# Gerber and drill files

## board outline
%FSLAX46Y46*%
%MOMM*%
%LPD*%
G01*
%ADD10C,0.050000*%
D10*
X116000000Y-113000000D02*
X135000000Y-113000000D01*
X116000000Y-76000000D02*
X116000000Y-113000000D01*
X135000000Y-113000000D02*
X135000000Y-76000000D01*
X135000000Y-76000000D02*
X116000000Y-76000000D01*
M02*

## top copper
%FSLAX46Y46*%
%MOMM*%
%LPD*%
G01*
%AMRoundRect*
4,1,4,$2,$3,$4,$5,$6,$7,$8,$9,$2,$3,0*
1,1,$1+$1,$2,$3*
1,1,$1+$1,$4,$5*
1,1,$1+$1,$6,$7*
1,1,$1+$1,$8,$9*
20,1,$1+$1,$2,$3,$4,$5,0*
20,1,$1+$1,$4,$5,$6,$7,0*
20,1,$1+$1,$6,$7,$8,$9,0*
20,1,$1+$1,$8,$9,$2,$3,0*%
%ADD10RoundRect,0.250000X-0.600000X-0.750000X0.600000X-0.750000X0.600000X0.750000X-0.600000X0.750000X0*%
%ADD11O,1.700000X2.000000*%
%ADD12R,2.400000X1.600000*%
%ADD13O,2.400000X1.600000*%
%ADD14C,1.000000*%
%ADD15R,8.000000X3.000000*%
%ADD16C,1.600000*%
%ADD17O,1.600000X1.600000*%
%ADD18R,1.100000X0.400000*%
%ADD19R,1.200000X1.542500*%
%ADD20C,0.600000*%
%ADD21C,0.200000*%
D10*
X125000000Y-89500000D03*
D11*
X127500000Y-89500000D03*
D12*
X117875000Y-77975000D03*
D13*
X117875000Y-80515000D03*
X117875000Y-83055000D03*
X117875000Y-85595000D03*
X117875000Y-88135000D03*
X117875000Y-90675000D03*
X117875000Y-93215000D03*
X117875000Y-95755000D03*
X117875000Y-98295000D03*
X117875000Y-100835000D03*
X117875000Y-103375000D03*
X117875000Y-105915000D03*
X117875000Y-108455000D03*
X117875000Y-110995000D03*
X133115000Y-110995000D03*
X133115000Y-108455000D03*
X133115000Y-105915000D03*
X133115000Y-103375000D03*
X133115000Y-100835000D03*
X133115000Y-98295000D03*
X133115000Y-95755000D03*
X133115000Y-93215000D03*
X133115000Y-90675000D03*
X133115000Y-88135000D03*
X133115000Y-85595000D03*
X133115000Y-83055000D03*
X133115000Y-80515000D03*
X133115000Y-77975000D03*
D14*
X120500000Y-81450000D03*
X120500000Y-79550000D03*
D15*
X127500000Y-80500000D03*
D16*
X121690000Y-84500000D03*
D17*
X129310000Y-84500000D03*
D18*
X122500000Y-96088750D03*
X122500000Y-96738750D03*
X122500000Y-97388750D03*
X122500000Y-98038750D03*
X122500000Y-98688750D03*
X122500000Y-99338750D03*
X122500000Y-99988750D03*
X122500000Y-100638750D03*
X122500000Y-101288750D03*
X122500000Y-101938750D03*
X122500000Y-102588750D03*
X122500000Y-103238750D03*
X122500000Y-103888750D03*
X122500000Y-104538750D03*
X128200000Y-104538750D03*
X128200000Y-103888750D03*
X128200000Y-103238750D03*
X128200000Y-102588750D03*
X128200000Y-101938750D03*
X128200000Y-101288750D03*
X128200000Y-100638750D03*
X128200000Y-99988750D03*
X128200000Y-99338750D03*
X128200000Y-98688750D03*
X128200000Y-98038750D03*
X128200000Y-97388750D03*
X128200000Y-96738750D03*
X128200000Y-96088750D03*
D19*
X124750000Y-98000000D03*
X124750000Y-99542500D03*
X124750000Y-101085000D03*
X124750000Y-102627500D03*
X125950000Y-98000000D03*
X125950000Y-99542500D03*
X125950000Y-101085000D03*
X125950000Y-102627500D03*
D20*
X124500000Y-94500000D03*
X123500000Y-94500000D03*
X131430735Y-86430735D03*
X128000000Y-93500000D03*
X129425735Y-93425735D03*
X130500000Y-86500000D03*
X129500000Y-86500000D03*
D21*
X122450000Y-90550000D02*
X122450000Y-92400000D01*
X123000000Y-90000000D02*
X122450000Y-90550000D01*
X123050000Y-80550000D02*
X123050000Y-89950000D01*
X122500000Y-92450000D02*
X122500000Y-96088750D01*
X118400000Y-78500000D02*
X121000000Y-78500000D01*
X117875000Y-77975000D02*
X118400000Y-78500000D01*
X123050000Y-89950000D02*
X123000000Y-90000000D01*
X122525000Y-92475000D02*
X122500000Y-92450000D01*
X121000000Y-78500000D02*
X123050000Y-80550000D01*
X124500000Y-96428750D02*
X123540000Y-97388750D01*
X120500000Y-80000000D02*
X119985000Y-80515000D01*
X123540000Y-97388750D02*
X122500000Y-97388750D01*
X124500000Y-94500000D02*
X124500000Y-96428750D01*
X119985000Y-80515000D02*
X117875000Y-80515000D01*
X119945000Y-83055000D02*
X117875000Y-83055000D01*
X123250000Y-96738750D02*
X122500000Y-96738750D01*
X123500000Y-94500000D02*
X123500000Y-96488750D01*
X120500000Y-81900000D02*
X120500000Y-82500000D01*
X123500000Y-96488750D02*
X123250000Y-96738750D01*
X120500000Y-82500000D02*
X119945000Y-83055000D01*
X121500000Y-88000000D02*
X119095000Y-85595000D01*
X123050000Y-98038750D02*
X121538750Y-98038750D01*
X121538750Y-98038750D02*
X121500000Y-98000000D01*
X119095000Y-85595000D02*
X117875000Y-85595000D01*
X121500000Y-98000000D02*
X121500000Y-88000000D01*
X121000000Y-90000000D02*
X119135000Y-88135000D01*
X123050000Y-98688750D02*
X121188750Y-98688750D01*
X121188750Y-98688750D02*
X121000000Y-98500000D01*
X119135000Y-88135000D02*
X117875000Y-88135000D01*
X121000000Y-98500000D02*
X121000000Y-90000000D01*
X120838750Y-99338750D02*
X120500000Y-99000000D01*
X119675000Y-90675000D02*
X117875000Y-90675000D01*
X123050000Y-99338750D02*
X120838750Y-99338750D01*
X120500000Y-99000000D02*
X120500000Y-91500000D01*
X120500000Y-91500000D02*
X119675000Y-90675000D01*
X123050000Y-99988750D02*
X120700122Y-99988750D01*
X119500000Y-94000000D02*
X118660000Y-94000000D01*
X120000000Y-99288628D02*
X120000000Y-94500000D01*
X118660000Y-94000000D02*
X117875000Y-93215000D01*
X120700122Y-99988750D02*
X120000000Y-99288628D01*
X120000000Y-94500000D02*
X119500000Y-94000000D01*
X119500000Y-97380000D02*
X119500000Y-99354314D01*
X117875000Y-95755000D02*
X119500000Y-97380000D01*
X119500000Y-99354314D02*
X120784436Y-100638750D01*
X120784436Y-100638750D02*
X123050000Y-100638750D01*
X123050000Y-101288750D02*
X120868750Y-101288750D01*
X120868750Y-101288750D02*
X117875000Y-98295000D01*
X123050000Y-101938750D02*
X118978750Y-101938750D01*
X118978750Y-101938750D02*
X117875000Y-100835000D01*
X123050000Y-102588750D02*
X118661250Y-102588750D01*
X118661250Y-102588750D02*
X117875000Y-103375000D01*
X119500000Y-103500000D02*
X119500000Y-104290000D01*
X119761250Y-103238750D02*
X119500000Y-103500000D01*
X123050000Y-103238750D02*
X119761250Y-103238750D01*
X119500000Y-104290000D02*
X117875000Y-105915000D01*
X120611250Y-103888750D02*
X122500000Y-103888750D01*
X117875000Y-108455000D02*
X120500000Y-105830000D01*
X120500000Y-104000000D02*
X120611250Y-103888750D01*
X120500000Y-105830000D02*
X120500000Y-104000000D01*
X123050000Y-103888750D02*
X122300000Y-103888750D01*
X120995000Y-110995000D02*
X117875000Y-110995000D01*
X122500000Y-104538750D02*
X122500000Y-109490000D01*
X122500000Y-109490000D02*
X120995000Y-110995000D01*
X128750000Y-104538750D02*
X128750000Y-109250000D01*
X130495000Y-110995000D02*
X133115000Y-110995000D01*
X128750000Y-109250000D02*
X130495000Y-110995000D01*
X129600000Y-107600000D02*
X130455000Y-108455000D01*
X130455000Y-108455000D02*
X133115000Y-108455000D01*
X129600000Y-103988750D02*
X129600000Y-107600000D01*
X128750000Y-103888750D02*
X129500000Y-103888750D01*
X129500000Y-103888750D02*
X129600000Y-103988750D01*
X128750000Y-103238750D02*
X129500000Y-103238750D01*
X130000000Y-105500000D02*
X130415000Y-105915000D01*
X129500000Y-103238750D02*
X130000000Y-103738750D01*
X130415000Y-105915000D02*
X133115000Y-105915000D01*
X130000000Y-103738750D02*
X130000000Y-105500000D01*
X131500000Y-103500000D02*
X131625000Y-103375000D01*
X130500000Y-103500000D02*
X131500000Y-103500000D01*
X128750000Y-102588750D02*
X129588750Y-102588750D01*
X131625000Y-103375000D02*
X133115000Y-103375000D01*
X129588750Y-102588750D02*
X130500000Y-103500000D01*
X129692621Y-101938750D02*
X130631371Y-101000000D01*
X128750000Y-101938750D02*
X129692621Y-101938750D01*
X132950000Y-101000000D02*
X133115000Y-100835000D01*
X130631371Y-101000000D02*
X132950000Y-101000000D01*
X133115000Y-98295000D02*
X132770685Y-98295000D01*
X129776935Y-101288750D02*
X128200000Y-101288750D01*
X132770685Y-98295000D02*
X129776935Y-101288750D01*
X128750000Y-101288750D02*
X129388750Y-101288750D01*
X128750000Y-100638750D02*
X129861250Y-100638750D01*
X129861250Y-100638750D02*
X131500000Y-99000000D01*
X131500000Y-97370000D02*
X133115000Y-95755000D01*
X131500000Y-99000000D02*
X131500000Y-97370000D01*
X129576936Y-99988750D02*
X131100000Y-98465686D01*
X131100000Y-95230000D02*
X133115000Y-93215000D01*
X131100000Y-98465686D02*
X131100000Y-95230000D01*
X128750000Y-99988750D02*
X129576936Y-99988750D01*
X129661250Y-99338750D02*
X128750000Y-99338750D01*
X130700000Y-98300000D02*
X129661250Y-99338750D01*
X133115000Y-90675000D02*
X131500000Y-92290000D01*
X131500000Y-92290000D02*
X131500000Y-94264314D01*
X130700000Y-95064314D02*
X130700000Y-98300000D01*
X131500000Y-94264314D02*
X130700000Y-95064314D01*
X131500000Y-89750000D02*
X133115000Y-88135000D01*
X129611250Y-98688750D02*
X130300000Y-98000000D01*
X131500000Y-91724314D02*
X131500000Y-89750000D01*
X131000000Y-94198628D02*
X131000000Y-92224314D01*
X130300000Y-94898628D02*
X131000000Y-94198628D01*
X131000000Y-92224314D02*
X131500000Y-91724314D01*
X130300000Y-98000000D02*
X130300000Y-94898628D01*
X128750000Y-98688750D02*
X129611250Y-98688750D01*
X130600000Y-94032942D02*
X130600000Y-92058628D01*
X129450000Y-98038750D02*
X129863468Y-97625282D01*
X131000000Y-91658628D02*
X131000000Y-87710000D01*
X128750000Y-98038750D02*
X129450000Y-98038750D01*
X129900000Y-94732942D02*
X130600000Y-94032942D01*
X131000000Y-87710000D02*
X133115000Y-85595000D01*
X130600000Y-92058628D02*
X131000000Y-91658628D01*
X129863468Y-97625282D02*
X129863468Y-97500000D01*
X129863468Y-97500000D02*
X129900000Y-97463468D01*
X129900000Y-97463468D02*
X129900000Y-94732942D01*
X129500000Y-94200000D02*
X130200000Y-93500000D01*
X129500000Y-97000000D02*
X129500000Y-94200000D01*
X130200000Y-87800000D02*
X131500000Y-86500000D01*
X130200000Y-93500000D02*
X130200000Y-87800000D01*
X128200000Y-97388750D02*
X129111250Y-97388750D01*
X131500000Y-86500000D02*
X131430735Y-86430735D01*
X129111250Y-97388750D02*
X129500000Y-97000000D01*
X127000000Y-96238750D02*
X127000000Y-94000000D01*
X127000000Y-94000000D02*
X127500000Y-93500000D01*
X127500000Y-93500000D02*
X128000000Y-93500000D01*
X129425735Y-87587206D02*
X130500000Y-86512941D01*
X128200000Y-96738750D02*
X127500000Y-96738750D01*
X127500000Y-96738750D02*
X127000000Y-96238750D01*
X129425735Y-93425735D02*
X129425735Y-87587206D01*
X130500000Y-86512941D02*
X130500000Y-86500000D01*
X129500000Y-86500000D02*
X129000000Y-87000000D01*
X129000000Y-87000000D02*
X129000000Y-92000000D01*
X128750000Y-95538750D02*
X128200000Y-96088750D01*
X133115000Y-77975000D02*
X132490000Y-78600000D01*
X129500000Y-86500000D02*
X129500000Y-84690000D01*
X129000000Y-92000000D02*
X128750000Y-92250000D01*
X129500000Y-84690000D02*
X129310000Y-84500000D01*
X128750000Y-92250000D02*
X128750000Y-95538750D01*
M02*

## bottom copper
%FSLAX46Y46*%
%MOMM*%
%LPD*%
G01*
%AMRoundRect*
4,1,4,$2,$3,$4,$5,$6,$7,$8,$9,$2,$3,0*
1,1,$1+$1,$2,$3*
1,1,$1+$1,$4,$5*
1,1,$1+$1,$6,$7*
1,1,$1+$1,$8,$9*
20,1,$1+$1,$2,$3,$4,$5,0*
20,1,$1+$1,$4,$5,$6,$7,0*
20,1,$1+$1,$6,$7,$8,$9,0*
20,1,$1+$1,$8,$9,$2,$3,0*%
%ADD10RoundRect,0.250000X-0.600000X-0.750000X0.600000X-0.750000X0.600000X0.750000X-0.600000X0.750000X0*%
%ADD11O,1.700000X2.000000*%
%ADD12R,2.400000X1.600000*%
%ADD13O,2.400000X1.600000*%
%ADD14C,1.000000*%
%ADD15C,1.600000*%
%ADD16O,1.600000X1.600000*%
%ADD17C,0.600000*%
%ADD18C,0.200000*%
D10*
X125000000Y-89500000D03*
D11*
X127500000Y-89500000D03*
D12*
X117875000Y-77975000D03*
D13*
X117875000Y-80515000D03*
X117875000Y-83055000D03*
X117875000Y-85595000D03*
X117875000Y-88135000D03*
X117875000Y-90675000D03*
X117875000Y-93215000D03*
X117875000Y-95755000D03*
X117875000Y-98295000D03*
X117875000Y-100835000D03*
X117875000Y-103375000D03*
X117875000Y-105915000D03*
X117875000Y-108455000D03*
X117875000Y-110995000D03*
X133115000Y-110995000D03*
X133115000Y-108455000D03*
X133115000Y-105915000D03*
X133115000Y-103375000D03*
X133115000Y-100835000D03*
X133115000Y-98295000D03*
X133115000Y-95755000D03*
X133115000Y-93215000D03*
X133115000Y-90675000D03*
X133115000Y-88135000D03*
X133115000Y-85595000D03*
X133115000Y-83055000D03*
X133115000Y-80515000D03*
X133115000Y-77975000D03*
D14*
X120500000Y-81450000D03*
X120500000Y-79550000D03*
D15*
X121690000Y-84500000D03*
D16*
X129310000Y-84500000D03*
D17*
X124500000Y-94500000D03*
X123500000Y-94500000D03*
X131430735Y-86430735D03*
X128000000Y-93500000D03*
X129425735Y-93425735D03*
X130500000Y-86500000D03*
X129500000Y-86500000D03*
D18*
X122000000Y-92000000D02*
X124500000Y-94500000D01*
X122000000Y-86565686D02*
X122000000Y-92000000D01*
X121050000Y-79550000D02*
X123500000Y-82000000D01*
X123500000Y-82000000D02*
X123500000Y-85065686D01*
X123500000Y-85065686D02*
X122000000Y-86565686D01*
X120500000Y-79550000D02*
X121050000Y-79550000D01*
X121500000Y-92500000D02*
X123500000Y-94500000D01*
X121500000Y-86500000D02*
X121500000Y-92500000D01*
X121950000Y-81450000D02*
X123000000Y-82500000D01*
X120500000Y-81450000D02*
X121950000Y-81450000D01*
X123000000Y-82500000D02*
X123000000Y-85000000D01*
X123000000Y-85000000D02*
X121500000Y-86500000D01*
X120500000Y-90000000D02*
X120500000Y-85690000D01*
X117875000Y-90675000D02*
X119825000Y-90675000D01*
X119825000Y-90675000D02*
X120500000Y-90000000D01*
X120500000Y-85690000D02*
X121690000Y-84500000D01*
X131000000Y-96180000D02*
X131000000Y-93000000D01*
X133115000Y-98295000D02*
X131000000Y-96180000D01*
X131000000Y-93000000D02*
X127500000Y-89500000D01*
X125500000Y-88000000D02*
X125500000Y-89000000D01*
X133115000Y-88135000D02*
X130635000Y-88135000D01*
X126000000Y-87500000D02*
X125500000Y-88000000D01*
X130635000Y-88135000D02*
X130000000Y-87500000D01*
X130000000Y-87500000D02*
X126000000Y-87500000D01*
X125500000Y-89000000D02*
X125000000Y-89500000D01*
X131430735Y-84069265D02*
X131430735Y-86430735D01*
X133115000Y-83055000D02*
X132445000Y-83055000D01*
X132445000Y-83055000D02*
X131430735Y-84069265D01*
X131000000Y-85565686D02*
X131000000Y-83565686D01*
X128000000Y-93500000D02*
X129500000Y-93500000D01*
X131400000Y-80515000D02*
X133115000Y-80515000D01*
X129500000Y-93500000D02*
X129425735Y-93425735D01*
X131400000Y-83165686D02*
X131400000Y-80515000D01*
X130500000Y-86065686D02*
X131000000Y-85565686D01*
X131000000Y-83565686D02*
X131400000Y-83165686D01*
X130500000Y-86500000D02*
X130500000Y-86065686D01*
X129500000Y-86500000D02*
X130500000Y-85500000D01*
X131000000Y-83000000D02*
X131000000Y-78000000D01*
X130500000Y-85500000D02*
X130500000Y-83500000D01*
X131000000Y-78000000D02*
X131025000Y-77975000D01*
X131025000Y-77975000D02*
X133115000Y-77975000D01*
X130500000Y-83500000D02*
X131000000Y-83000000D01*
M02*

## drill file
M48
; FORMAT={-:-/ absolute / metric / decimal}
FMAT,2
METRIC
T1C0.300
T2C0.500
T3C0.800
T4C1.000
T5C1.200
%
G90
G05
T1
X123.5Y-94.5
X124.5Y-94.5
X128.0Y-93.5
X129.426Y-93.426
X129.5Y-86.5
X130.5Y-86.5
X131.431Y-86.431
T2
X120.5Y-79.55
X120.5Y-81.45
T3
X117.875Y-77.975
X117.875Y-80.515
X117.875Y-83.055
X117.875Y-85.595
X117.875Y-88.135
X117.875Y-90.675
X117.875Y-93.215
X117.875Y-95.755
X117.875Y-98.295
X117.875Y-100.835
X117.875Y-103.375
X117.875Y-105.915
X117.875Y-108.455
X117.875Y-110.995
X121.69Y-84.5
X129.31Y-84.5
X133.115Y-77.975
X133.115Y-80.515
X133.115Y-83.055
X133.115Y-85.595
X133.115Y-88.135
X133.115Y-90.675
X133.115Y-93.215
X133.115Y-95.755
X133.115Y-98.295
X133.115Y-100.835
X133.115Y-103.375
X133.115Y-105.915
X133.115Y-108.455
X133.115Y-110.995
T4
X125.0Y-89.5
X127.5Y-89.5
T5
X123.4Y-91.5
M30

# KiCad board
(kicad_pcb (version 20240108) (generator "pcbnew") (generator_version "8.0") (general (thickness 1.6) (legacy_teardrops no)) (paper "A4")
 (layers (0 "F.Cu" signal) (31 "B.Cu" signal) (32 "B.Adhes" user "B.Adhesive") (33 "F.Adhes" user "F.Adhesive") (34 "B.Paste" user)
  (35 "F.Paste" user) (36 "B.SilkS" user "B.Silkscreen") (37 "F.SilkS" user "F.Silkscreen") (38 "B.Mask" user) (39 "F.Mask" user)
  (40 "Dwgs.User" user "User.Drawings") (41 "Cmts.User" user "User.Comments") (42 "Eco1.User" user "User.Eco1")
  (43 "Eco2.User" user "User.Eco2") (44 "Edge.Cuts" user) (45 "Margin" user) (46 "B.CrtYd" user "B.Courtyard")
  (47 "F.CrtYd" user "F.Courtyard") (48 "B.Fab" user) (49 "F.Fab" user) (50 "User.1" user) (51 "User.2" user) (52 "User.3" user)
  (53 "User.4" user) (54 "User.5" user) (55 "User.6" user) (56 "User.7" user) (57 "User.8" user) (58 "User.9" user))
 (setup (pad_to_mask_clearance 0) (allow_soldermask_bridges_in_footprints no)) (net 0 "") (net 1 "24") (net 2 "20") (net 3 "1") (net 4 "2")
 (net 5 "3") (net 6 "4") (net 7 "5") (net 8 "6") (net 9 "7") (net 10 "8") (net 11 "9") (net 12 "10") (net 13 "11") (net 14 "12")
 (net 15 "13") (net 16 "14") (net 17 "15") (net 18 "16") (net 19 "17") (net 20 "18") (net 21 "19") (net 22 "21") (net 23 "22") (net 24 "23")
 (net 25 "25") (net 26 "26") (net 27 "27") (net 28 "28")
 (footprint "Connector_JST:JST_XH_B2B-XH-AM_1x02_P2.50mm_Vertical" (layer "F.Cu") (at 125 89.5)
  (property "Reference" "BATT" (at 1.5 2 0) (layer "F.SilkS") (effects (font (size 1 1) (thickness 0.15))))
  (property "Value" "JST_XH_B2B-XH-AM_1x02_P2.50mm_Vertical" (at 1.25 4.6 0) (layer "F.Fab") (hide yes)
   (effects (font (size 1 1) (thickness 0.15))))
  (pad "" np_thru_hole circle (at -1.6 2) (size 1.2 1.2) (drill 1.2) (layers "*.Cu" "*.Mask"))
  (pad "1" thru_hole roundrect (at 0 0) (size 1.7 2) (drill 1) (layers "*.Cu" "*.Mask") (remove_unused_layers no)
   (roundrect_rratio 0.147059) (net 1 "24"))
  (pad "2" thru_hole oval (at 2.5 0) (size 1.7 2) (drill 1) (layers "*.Cu" "*.Mask") (remove_unused_layers no) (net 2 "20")))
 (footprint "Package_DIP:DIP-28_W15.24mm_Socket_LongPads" (layer "F.Cu") (at 117.875 77.975)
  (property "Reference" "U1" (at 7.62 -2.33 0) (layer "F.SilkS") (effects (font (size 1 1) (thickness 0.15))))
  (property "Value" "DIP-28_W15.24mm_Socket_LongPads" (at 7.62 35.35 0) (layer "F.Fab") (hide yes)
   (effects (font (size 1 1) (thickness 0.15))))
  (pad "1" thru_hole rect (at 0 0) (size 2.4 1.6) (drill 0.8) (layers "*.Cu" "*.Mask") (remove_unused_layers no) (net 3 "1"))
  (pad "2" thru_hole oval (at 0 2.54) (size 2.4 1.6) (drill 0.8) (layers "*.Cu" "*.Mask") (remove_unused_layers no) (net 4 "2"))
  (pad "3" thru_hole oval (at 0 5.08) (size 2.4 1.6) (drill 0.8) (layers "*.Cu" "*.Mask") (remove_unused_layers no) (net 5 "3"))
  (pad "4" thru_hole oval (at 0 7.62) (size 2.4 1.6) (drill 0.8) (layers "*.Cu" "*.Mask") (remove_unused_layers no) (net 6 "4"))
  (pad "5" thru_hole oval (at 0 10.16) (size 2.4 1.6) (drill 0.8) (layers "*.Cu" "*.Mask") (remove_unused_layers no) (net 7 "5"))
  (pad "6" thru_hole oval (at 0 12.7) (size 2.4 1.6) (drill 0.8) (layers "*.Cu" "*.Mask") (remove_unused_layers no) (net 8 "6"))
  (pad "7" thru_hole oval (at 0 15.24) (size 2.4 1.6) (drill 0.8) (layers "*.Cu" "*.Mask") (remove_unused_layers no) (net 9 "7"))
  (pad "8" thru_hole oval (at 0 17.78) (size 2.4 1.6) (drill 0.8) (layers "*.Cu" "*.Mask") (remove_unused_layers no) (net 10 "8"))
  (pad "9" thru_hole oval (at 0 20.32) (size 2.4 1.6) (drill 0.8) (layers "*.Cu" "*.Mask") (remove_unused_layers no) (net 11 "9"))
  (pad "10" thru_hole oval (at 0 22.86) (size 2.4 1.6) (drill 0.8) (layers "*.Cu" "*.Mask") (remove_unused_layers no) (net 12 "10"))
  (pad "11" thru_hole oval (at 0 25.4) (size 2.4 1.6) (drill 0.8) (layers "*.Cu" "*.Mask") (remove_unused_layers no) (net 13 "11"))
  (pad "12" thru_hole oval (at 0 27.94) (size 2.4 1.6) (drill 0.8) (layers "*.Cu" "*.Mask") (remove_unused_layers no) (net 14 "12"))
  (pad "13" thru_hole oval (at 0 30.48) (size 2.4 1.6) (drill 0.8) (layers "*.Cu" "*.Mask") (remove_unused_layers no) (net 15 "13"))
  (pad "14" thru_hole oval (at 0 33.02) (size 2.4 1.6) (drill 0.8) (layers "*.Cu" "*.Mask") (remove_unused_layers no) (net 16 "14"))
  (pad "15" thru_hole oval (at 15.24 33.02) (size 2.4 1.6) (drill 0.8) (layers "*.Cu" "*.Mask") (remove_unused_layers no) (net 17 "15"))
  (pad "16" thru_hole oval (at 15.24 30.48) (size 2.4 1.6) (drill 0.8) (layers "*.Cu" "*.Mask") (remove_unused_layers no) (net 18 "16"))
  (pad "17" thru_hole oval (at 15.24 27.94) (size 2.4 1.6) (drill 0.8) (layers "*.Cu" "*.Mask") (remove_unused_layers no) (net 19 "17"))
  (pad "18" thru_hole oval (at 15.24 25.4) (size 2.4 1.6) (drill 0.8) (layers "*.Cu" "*.Mask") (remove_unused_layers no) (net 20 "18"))
  (pad "19" thru_hole oval (at 15.24 22.86) (size 2.4 1.6) (drill 0.8) (layers "*.Cu" "*.Mask") (remove_unused_layers no) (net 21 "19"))
  (pad "20" thru_hole oval (at 15.24 20.32) (size 2.4 1.6) (drill 0.8) (layers "*.Cu" "*.Mask") (remove_unused_layers no) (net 2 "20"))
  (pad "21" thru_hole oval (at 15.24 17.78) (size 2.4 1.6) (drill 0.8) (layers "*.Cu" "*.Mask") (remove_unused_layers no) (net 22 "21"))
  (pad "22" thru_hole oval (at 15.24 15.24) (size 2.4 1.6) (drill 0.8) (layers "*.Cu" "*.Mask") (remove_unused_layers no) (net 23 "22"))
  (pad "23" thru_hole oval (at 15.24 12.7) (size 2.4 1.6) (drill 0.8) (layers "*.Cu" "*.Mask") (remove_unused_layers no) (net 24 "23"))
  (pad "24" thru_hole oval (at 15.24 10.16) (size 2.4 1.6) (drill 0.8) (layers "*.Cu" "*.Mask") (remove_unused_layers no) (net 1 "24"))
  (pad "25" thru_hole oval (at 15.24 7.62) (size 2.4 1.6) (drill 0.8) (layers "*.Cu" "*.Mask") (remove_unused_layers no) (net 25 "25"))
  (pad "26" thru_hole oval (at 15.24 5.08) (size 2.4 1.6) (drill 0.8) (layers "*.Cu" "*.Mask") (remove_unused_layers no) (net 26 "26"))
  (pad "27" thru_hole oval (at 15.24 2.54) (size 2.4 1.6) (drill 0.8) (layers "*.Cu" "*.Mask") (remove_unused_layers no) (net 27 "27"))
  (pad "28" thru_hole oval (at 15.24 0) (size 2.4 1.6) (drill 0.8) (layers "*.Cu" "*.Mask") (remove_unused_layers no) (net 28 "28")))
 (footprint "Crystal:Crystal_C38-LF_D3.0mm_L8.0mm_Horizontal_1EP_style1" (layer "F.Cu") (at 120.5 81.45 90)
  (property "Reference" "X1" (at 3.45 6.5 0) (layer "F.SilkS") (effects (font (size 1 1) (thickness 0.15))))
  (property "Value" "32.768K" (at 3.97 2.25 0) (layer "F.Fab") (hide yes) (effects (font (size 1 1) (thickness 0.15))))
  (pad "1" thru_hole circle (at 0 0 90) (size 1 1) (drill 0.5) (layers "*.Cu" "*.Mask") (remove_unused_layers no) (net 5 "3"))
  (pad "2" thru_hole circle (at 1.9 0 90) (size 1 1) (drill 0.5) (layers "*.Cu" "*.Mask") (remove_unused_layers no) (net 4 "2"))
  (pad "3" smd rect (at 0.95 7 90) (size 3 8) (layers "F.Cu")))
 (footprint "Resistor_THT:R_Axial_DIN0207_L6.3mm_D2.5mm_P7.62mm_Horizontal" (layer "F.Cu") (at 121.69 84.5)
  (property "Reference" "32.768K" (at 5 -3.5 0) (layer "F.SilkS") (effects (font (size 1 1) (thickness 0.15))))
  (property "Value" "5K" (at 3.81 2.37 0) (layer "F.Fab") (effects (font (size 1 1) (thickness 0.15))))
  (pad "1" thru_hole circle (at 0 0) (size 1.6 1.6) (drill 0.8) (layers "*.Cu" "*.Mask") (remove_unused_layers no) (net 8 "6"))
  (pad "2" thru_hole oval (at 7.62 0) (size 1.6 1.6) (drill 0.8) (layers "*.Cu" "*.Mask") (remove_unused_layers no) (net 28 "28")))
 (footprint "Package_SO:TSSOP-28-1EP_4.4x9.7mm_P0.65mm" (layer "F.Cu") (at 125.35 100.31375)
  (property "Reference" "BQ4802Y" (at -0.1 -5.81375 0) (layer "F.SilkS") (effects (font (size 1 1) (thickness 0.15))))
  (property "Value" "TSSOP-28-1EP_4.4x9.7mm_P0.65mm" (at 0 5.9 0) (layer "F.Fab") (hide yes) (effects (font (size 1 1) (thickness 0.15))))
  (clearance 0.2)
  (pad "1" smd rect (at -2.85 -4.225) (size 1.1 0.4) (layers "F.Cu" "F.Paste" "F.Mask") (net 3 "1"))
  (pad "2" smd rect (at -2.85 -3.575) (size 1.1 0.4) (layers "F.Cu" "F.Paste" "F.Mask") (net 5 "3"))
  (pad "3" smd rect (at -2.85 -2.925) (size 1.1 0.4) (layers "F.Cu" "F.Paste" "F.Mask") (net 4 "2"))
  (pad "4" smd rect (at -2.85 -2.275) (size 1.1 0.4) (layers "F.Cu" "F.Paste" "F.Mask") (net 6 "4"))
  (pad "5" smd rect (at -2.85 -1.625) (size 1.1 0.4) (layers "F.Cu" "F.Paste" "F.Mask") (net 7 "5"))
  (pad "6" smd rect (at -2.85 -0.975) (size 1.1 0.4) (layers "F.Cu" "F.Paste" "F.Mask") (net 8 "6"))
  (pad "7" smd rect (at -2.85 -0.325) (size 1.1 0.4) (layers "F.Cu" "F.Paste" "F.Mask") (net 9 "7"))
  (pad "8" smd rect (at -2.85 0.325) (size 1.1 0.4) (layers "F.Cu" "F.Paste" "F.Mask") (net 10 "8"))
  (pad "9" smd rect (at -2.85 0.975) (size 1.1 0.4) (layers "F.Cu" "F.Paste" "F.Mask") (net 11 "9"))
  (pad "10" smd rect (at -2.85 1.625) (size 1.1 0.4) (layers "F.Cu" "F.Paste" "F.Mask") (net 12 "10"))
  (pad "11" smd rect (at -2.85 2.275) (size 1.1 0.4) (layers "F.Cu" "F.Paste" "F.Mask") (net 13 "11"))
  (pad "12" smd rect (at -2.85 2.925) (size 1.1 0.4) (layers "F.Cu" "F.Paste" "F.Mask") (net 14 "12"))
  (pad "13" smd rect (at -2.85 3.575) (size 1.1 0.4) (layers "F.Cu" "F.Paste" "F.Mask") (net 15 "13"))
  (pad "14" smd rect (at -2.85 4.225) (size 1.1 0.4) (layers "F.Cu" "F.Paste" "F.Mask") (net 16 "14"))
  (pad "15" smd rect (at 2.85 4.225) (size 1.1 0.4) (layers "F.Cu" "F.Paste" "F.Mask") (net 17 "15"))
  (pad "16" smd rect (at 2.85 3.575) (size 1.1 0.4) (layers "F.Cu" "F.Paste" "F.Mask") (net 18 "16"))
  (pad "17" smd rect (at 2.85 2.925) (size 1.1 0.4) (layers "F.Cu" "F.Paste" "F.Mask") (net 19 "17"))
  (pad "18" smd rect (at 2.85 2.275) (size 1.1 0.4) (layers "F.Cu" "F.Paste" "F.Mask") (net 20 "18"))
  (pad "19" smd rect (at 2.85 1.625) (size 1.1 0.4) (layers "F.Cu" "F.Paste" "F.Mask") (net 21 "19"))
  (pad "20" smd rect (at 2.85 0.975) (size 1.1 0.4) (layers "F.Cu" "F.Paste" "F.Mask") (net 2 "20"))
  (pad "21" smd rect (at 2.85 0.325) (size 1.1 0.4) (layers "F.Cu" "F.Paste" "F.Mask") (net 22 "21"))
  (pad "22" smd rect (at 2.85 -0.325) (size 1.1 0.4) (layers "F.Cu" "F.Paste" "F.Mask") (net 23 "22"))
  (pad "23" smd rect (at 2.85 -0.975) (size 1.1 0.4) (layers "F.Cu" "F.Paste" "F.Mask") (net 24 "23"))
  (pad "24" smd rect (at 2.85 -1.625) (size 1.1 0.4) (layers "F.Cu" "F.Paste" "F.Mask") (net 1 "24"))
  (pad "25" smd rect (at 2.85 -2.275) (size 1.1 0.4) (layers "F.Cu" "F.Paste" "F.Mask") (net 25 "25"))
  (pad "26" smd rect (at 2.85 -2.925) (size 1.1 0.4) (layers "F.Cu" "F.Paste" "F.Mask") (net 26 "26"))
  (pad "27" smd rect (at 2.85 -3.575) (size 1.1 0.4) (layers "F.Cu" "F.Paste" "F.Mask") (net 27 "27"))
  (pad "28" smd rect (at 2.85 -4.225) (size 1.1 0.4) (layers "F.Cu" "F.Paste" "F.Mask") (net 28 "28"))
  (pad "29" smd rect (at -0.6 -2.31375) (size 1.2 1.5425) (layers "F.Cu" "F.Paste" "F.Mask") (solder_paste_margin_ratio -0.2))
  (pad "29" smd rect (at -0.6 -0.77125) (size 1.2 1.5425) (layers "F.Cu" "F.Paste" "F.Mask") (solder_paste_margin_ratio -0.2))
  (pad "29" smd rect (at -0.6 0.77125) (size 1.2 1.5425) (layers "F.Cu" "F.Paste" "F.Mask") (solder_paste_margin_ratio -0.2))
  (pad "29" smd rect (at -0.6 2.31375) (size 1.2 1.5425) (layers "F.Cu" "F.Paste" "F.Mask") (solder_paste_margin_ratio -0.2))
  (pad "29" smd rect (at 0.6 -2.31375) (size 1.2 1.5425) (layers "F.Cu" "F.Paste" "F.Mask") (solder_paste_margin_ratio -0.2))
  (pad "29" smd rect (at 0.6 -0.77125) (size 1.2 1.5425) (layers "F.Cu" "F.Paste" "F.Mask") (solder_paste_margin_ratio -0.2))
  (pad "29" smd rect (at 0.6 0.77125) (size 1.2 1.5425) (layers "F.Cu" "F.Paste" "F.Mask") (solder_paste_margin_ratio -0.2))
  (pad "29" smd rect (at 0.6 2.31375) (size 1.2 1.5425) (layers "F.Cu" "F.Paste" "F.Mask") (solder_paste_margin_ratio -0.2)))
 (gr_line (start 116 113) (end 135 113) (stroke (width 0.05) (type default)) (layer "Edge.Cuts"))
 (gr_line (start 116 76) (end 116 113) (stroke (width 0.05) (type default)) (layer "Edge.Cuts"))
 (gr_line (start 135 113) (end 135 76) (stroke (width 0.05) (type default)) (layer "Edge.Cuts"))
 (gr_line (start 135 76) (end 116 76) (stroke (width 0.05) (type default)) (layer "Edge.Cuts"))
 (segment (start 122.45 90.55) (end 122.45 92.4) (width 0.2) (layer "F.Cu") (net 3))
 (segment (start 123 90) (end 122.45 90.55) (width 0.2) (layer "F.Cu") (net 3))
 (segment (start 123.05 80.55) (end 123.05 89.95) (width 0.2) (layer "F.Cu") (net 3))
 (segment (start 122.5 92.45) (end 122.5 96.08875) (width 0.2) (layer "F.Cu") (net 3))
 (segment (start 118.4 78.5) (end 121 78.5) (width 0.2) (layer "F.Cu") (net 3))
 (segment (start 117.875 77.975) (end 118.4 78.5) (width 0.2) (layer "F.Cu") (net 3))
 (segment (start 123.05 89.95) (end 123 90) (width 0.2) (layer "F.Cu") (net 3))
 (segment (start 122.525 92.475) (end 122.5 92.45) (width 0.2) (layer "F.Cu") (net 3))
 (segment (start 121 78.5) (end 123.05 80.55) (width 0.2) (layer "F.Cu") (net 3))
 (segment (start 124.5 96.42875) (end 123.54 97.38875) (width 0.2) (layer "F.Cu") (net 4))
 (segment (start 120.5 80) (end 119.985 80.515) (width 0.2) (layer "F.Cu") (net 4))
 (segment (start 123.54 97.38875) (end 122.5 97.38875) (width 0.2) (layer "F.Cu") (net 4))
 (segment (start 124.5 94.5) (end 124.5 96.42875) (width 0.2) (layer "F.Cu") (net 4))
 (segment (start 119.985 80.515) (end 117.875 80.515) (width 0.2) (layer "F.Cu") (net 4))
 (via (at 124.5 94.5) (size 0.6) (drill 0.3) (layers "F.Cu" "B.Cu") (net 4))
 (segment (start 122 92) (end 124.5 94.5) (width 0.2) (layer "B.Cu") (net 4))
 (segment (start 122 86.565686) (end 122 92) (width 0.2) (layer "B.Cu") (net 4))
 (segment (start 121.05 79.55) (end 123.5 82) (width 0.2) (layer "B.Cu") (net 4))
 (segment (start 123.5 82) (end 123.5 85.065686) (width 0.2) (layer "B.Cu") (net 4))
 (segment (start 123.5 85.065686) (end 122 86.565686) (width 0.2) (layer "B.Cu") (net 4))
 (segment (start 120.5 79.55) (end 121.05 79.55) (width 0.2) (layer "B.Cu") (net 4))
 (segment (start 119.945 83.055) (end 117.875 83.055) (width 0.2) (layer "F.Cu") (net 5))
 (segment (start 123.25 96.73875) (end 122.5 96.73875) (width 0.2) (layer "F.Cu") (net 5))
 (segment (start 123.5 94.5) (end 123.5 96.48875) (width 0.2) (layer "F.Cu") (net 5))
 (segment (start 120.5 81.9) (end 120.5 82.5) (width 0.2) (layer "F.Cu") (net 5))
 (segment (start 123.5 96.48875) (end 123.25 96.73875) (width 0.2) (layer "F.Cu") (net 5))
 (segment (start 120.5 82.5) (end 119.945 83.055) (width 0.2) (layer "F.Cu") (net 5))
 (via (at 123.5 94.5) (size 0.6) (drill 0.3) (layers "F.Cu" "B.Cu") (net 5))
 (segment (start 121.5 92.5) (end 123.5 94.5) (width 0.2) (layer "B.Cu") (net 5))
 (segment (start 121.5 86.5) (end 121.5 92.5) (width 0.2) (layer "B.Cu") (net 5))
 (segment (start 121.95 81.45) (end 123 82.5) (width 0.2) (layer "B.Cu") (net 5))
 (segment (start 120.5 81.45) (end 121.95 81.45) (width 0.2) (layer "B.Cu") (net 5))
 (segment (start 123 82.5) (end 123 85) (width 0.2) (layer "B.Cu") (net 5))
 (segment (start 123 85) (end 121.5 86.5) (width 0.2) (layer "B.Cu") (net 5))
 (segment (start 121.5 88) (end 119.095 85.595) (width 0.2) (layer "F.Cu") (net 6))
 (segment (start 123.05 98.03875) (end 121.53875 98.03875) (width 0.2) (layer "F.Cu") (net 6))
 (segment (start 121.53875 98.03875) (end 121.5 98) (width 0.2) (layer "F.Cu") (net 6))
 (segment (start 119.095 85.595) (end 117.875 85.595) (width 0.2) (layer "F.Cu") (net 6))
 (segment (start 121.5 98) (end 121.5 88) (width 0.2) (layer "F.Cu") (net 6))
 (segment (start 121 90) (end 119.135 88.135) (width 0.2) (layer "F.Cu") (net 7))
 (segment (start 123.05 98.68875) (end 121.18875 98.68875) (width 0.2) (layer "F.Cu") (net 7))
 (segment (start 121.18875 98.68875) (end 121 98.5) (width 0.2) (layer "F.Cu") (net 7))
 (segment (start 119.135 88.135) (end 117.875 88.135) (width 0.2) (layer "F.Cu") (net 7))
 (segment (start 121 98.5) (end 121 90) (width 0.2) (layer "F.Cu") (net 7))
 (segment (start 120.83875 99.33875) (end 120.5 99) (width 0.2) (layer "F.Cu") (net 8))
 (segment (start 119.675 90.675) (end 117.875 90.675) (width 0.2) (layer "F.Cu") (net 8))
 (segment (start 123.05 99.33875) (end 120.83875 99.33875) (width 0.2) (layer "F.Cu") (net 8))
 (segment (start 120.5 99) (end 120.5 91.5) (width 0.2) (layer "F.Cu") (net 8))
 (segment (start 120.5 91.5) (end 119.675 90.675) (width 0.2) (layer "F.Cu") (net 8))
 (segment (start 120.5 90) (end 120.5 85.69) (width 0.2) (layer "B.Cu") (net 8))
 (segment (start 117.875 90.675) (end 119.825 90.675) (width 0.2) (layer "B.Cu") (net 8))
 (segment (start 119.825 90.675) (end 120.5 90) (width 0.2) (layer "B.Cu") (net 8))
 (segment (start 120.5 85.69) (end 121.69 84.5) (width 0.2) (layer "B.Cu") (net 8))
 (segment (start 123.05 99.98875) (end 120.700122 99.98875) (width 0.2) (layer "F.Cu") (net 9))
 (segment (start 119.5 94) (end 118.66 94) (width 0.2) (layer "F.Cu") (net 9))
 (segment (start 120 99.288628) (end 120 94.5) (width 0.2) (layer "F.Cu") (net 9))
 (segment (start 118.66 94) (end 117.875 93.215) (width 0.2) (layer "F.Cu") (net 9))
 (segment (start 120.700122 99.98875) (end 120 99.288628) (width 0.2) (layer "F.Cu") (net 9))
 (segment (start 120 94.5) (end 119.5 94) (width 0.2) (layer "F.Cu") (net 9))
 (segment (start 119.5 97.38) (end 119.5 99.354314) (width 0.2) (layer "F.Cu") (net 10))
 (segment (start 117.875 95.755) (end 119.5 97.38) (width 0.2) (layer "F.Cu") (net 10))
 (segment (start 119.5 99.354314) (end 120.784436 100.63875) (width 0.2) (layer "F.Cu") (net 10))
 (segment (start 120.784436 100.63875) (end 123.05 100.63875) (width 0.2) (layer "F.Cu") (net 10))
 (segment (start 123.05 101.28875) (end 120.86875 101.28875) (width 0.2) (layer "F.Cu") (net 11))
 (segment (start 120.86875 101.28875) (end 117.875 98.295) (width 0.2) (layer "F.Cu") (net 11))
 (segment (start 123.05 101.93875) (end 118.97875 101.93875) (width 0.2) (layer "F.Cu") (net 12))
 (segment (start 118.97875 101.93875) (end 117.875 100.835) (width 0.2) (layer "F.Cu") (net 12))
 (segment (start 123.05 102.58875) (end 118.66125 102.58875) (width 0.2) (layer "F.Cu") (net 13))
 (segment (start 118.66125 102.58875) (end 117.875 103.375) (width 0.2) (layer "F.Cu") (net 13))
 (segment (start 119.5 103.5) (end 119.5 104.29) (width 0.2) (layer "F.Cu") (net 14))
 (segment (start 119.76125 103.23875) (end 119.5 103.5) (width 0.2) (layer "F.Cu") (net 14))
 (segment (start 123.05 103.23875) (end 119.76125 103.23875) (width 0.2) (layer "F.Cu") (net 14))
 (segment (start 119.5 104.29) (end 117.875 105.915) (width 0.2) (layer "F.Cu") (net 14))
 (segment (start 120.61125 103.88875) (end 122.5 103.88875) (width 0.2) (layer "F.Cu") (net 15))
 (segment (start 117.875 108.455) (end 120.5 105.83) (width 0.2) (layer "F.Cu") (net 15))
 (segment (start 120.5 104) (end 120.61125 103.88875) (width 0.2) (layer "F.Cu") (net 15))
 (segment (start 120.5 105.83) (end 120.5 104) (width 0.2) (layer "F.Cu") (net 15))
 (segment (start 123.05 103.88875) (end 122.3 103.88875) (width 0.2) (layer "F.Cu") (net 15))
 (segment (start 120.995 110.995) (end 117.875 110.995) (width 0.2) (layer "F.Cu") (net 16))
 (segment (start 122.5 104.53875) (end 122.5 109.49) (width 0.2) (layer "F.Cu") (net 16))
 (segment (start 122.5 109.49) (end 120.995 110.995) (width 0.2) (layer "F.Cu") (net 16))
 (segment (start 128.75 104.53875) (end 128.75 109.25) (width 0.2) (layer "F.Cu") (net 17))
 (segment (start 130.495 110.995) (end 133.115 110.995) (width 0.2) (layer "F.Cu") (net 17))
 (segment (start 128.75 109.25) (end 130.495 110.995) (width 0.2) (layer "F.Cu") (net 17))
 (segment (start 129.6 107.6) (end 130.455 108.455) (width 0.2) (layer "F.Cu") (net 18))
 (segment (start 130.455 108.455) (end 133.115 108.455) (width 0.2) (layer "F.Cu") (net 18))
 (segment (start 129.6 103.98875) (end 129.6 107.6) (width 0.2) (layer "F.Cu") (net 18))
 (segment (start 128.75 103.88875) (end 129.5 103.88875) (width 0.2) (layer "F.Cu") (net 18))
 (segment (start 129.5 103.88875) (end 129.6 103.98875) (width 0.2) (layer "F.Cu") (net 18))
 (segment (start 128.75 103.23875) (end 129.5 103.23875) (width 0.2) (layer "F.Cu") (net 19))
 (segment (start 130 105.5) (end 130.415 105.915) (width 0.2) (layer "F.Cu") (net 19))
 (segment (start 129.5 103.23875) (end 130 103.73875) (width 0.2) (layer "F.Cu") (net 19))
 (segment (start 130.415 105.915) (end 133.115 105.915) (width 0.2) (layer "F.Cu") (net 19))
 (segment (start 130 103.73875) (end 130 105.5) (width 0.2) (layer "F.Cu") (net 19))
 (segment (start 131.5 103.5) (end 131.625 103.375) (width 0.2) (layer "F.Cu") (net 20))
 (segment (start 130.5 103.5) (end 131.5 103.5) (width 0.2) (layer "F.Cu") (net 20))
 (segment (start 128.75 102.58875) (end 129.58875 102.58875) (width 0.2) (layer "F.Cu") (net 20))
 (segment (start 131.625 103.375) (end 133.115 103.375) (width 0.2) (layer "F.Cu") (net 20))
 (segment (start 129.58875 102.58875) (end 130.5 103.5) (width 0.2) (layer "F.Cu") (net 20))
 (segment (start 129.692621 101.93875) (end 130.631371 101) (width 0.2) (layer "F.Cu") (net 21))
 (segment (start 128.75 101.93875) (end 129.692621 101.93875) (width 0.2) (layer "F.Cu") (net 21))
 (segment (start 132.95 101) (end 133.115 100.835) (width 0.2) (layer "F.Cu") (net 21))
 (segment (start 130.631371 101) (end 132.95 101) (width 0.2) (layer "F.Cu") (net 21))
 (segment (start 133.115 98.295) (end 132.770685 98.295) (width 0.2) (layer "F.Cu") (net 2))
 (segment (start 129.776935 101.28875) (end 128.2 101.28875) (width 0.2) (layer "F.Cu") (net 2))
 (segment (start 132.770685 98.295) (end 129.776935 101.28875) (width 0.2) (layer "F.Cu") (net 2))
 (segment (start 128.75 101.28875) (end 129.38875 101.28875) (width 0.2) (layer "F.Cu") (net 2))
 (segment (start 131 96.18) (end 131 93) (width 0.2) (layer "B.Cu") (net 2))
 (segment (start 133.115 98.295) (end 131 96.18) (width 0.2) (layer "B.Cu") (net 2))
 (segment (start 131 93) (end 127.5 89.5) (width 0.2) (layer "B.Cu") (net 2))
 (segment (start 128.75 100.63875) (end 129.86125 100.63875) (width 0.2) (layer "F.Cu") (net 22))
 (segment (start 129.86125 100.63875) (end 131.5 99) (width 0.2) (layer "F.Cu") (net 22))
 (segment (start 131.5 97.37) (end 133.115 95.755) (width 0.2) (layer "F.Cu") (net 22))
 (segment (start 131.5 99) (end 131.5 97.37) (width 0.2) (layer "F.Cu") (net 22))
 (segment (start 129.576936 99.98875) (end 131.1 98.465686) (width 0.2) (layer "F.Cu") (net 23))
 (segment (start 131.1 95.23) (end 133.115 93.215) (width 0.2) (layer "F.Cu") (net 23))
 (segment (start 131.1 98.465686) (end 131.1 95.23) (width 0.2) (layer "F.Cu") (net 23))
 (segment (start 128.75 99.98875) (end 129.576936 99.98875) (width 0.2) (layer "F.Cu") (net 23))
 (segment (start 129.66125 99.33875) (end 128.75 99.33875) (width 0.2) (layer "F.Cu") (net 24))
 (segment (start 130.7 98.3) (end 129.66125 99.33875) (width 0.2) (layer "F.Cu") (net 24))
 (segment (start 133.115 90.675) (end 131.5 92.29) (width 0.2) (layer "F.Cu") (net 24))
 (segment (start 131.5 92.29) (end 131.5 94.264314) (width 0.2) (layer "F.Cu") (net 24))
 (segment (start 130.7 95.064314) (end 130.7 98.3) (width 0.2) (layer "F.Cu") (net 24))
 (segment (start 131.5 94.264314) (end 130.7 95.064314) (width 0.2) (layer "F.Cu") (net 24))
 (segment (start 131.5 89.75) (end 133.115 88.135) (width 0.2) (layer "F.Cu") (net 1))
 (segment (start 129.61125 98.68875) (end 130.3 98) (width 0.2) (layer "F.Cu") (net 1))
 (segment (start 131.5 91.724314) (end 131.5 89.75) (width 0.2) (layer "F.Cu") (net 1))
 (segment (start 131 94.198628) (end 131 92.224314) (width 0.2) (layer "F.Cu") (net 1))
 (segment (start 130.3 94.898628) (end 131 94.198628) (width 0.2) (layer "F.Cu") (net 1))
 (segment (start 131 92.224314) (end 131.5 91.724314) (width 0.2) (layer "F.Cu") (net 1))
 (segment (start 130.3 98) (end 130.3 94.898628) (width 0.2) (layer "F.Cu") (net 1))
 (segment (start 128.75 98.68875) (end 129.61125 98.68875) (width 0.2) (layer "F.Cu") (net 1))
 (segment (start 125.5 88) (end 125.5 89) (width 0.2) (layer "B.Cu") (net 1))
 (segment (start 133.115 88.135) (end 130.635 88.135) (width 0.2) (layer "B.Cu") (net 1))
 (segment (start 126 87.5) (end 125.5 88) (width 0.2) (layer "B.Cu") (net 1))
 (segment (start 130.635 88.135) (end 130 87.5) (width 0.2) (layer "B.Cu") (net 1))
 (segment (start 130 87.5) (end 126 87.5) (width 0.2) (layer "B.Cu") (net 1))
 (segment (start 125.5 89) (end 125 89.5) (width 0.2) (layer "B.Cu") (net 1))
 (segment (start 130.6 94.032942) (end 130.6 92.058628) (width 0.2) (layer "F.Cu") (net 25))
 (segment (start 129.45 98.03875) (end 129.863468 97.625282) (width 0.2) (layer "F.Cu") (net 25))
 (segment (start 131 91.658628) (end 131 87.71) (width 0.2) (layer "F.Cu") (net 25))
 (segment (start 128.75 98.03875) (end 129.45 98.03875) (width 0.2) (layer "F.Cu") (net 25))
 (segment (start 129.9 94.732942) (end 130.6 94.032942) (width 0.2) (layer "F.Cu") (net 25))
 (segment (start 131 87.71) (end 133.115 85.595) (width 0.2) (layer "F.Cu") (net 25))
 (segment (start 130.6 92.058628) (end 131 91.658628) (width 0.2) (layer "F.Cu") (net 25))
 (segment (start 129.863468 97.625282) (end 129.863468 97.5) (width 0.2) (layer "F.Cu") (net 25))
 (segment (start 129.863468 97.5) (end 129.9 97.463468) (width 0.2) (layer "F.Cu") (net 25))
 (segment (start 129.9 97.463468) (end 129.9 94.732942) (width 0.2) (layer "F.Cu") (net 25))
 (segment (start 129.5 94.2) (end 130.2 93.5) (width 0.2) (layer "F.Cu") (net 26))
 (segment (start 129.5 97) (end 129.5 94.2) (width 0.2) (layer "F.Cu") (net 26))
 (segment (start 130.2 87.8) (end 131.5 86.5) (width 0.2) (layer "F.Cu") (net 26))
 (segment (start 130.2 93.5) (end 130.2 87.8) (width 0.2) (layer "F.Cu") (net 26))
 (segment (start 128.2 97.38875) (end 129.11125 97.38875) (width 0.2) (layer "F.Cu") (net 26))
 (segment (start 131.5 86.5) (end 131.430735 86.430735) (width 0.2) (layer "F.Cu") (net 26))
 (segment (start 129.11125 97.38875) (end 129.5 97) (width 0.2) (layer "F.Cu") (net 26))
 (via (at 131.430735 86.430735) (size 0.6) (drill 0.3) (layers "F.Cu" "B.Cu") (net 26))
 (segment (start 131.430735 84.069265) (end 131.430735 86.430735) (width 0.2) (layer "B.Cu") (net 26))
 (segment (start 133.115 83.055) (end 132.445 83.055) (width 0.2) (layer "B.Cu") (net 26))
 (segment (start 132.445 83.055) (end 131.430735 84.069265) (width 0.2) (layer "B.Cu") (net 26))
 (segment (start 127 96.23875) (end 127 94) (width 0.2) (layer "F.Cu") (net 27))
 (segment (start 127 94) (end 127.5 93.5) (width 0.2) (layer "F.Cu") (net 27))
 (segment (start 127.5 93.5) (end 128 93.5) (width 0.2) (layer "F.Cu") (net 27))
 (segment (start 129.425735 87.587206) (end 130.5 86.512941) (width 0.2) (layer "F.Cu") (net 27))
 (segment (start 128.2 96.73875) (end 127.5 96.73875) (width 0.2) (layer "F.Cu") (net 27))
 (segment (start 127.5 96.73875) (end 127 96.23875) (width 0.2) (layer "F.Cu") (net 27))
 (segment (start 129.425735 93.425735) (end 129.425735 87.587206) (width 0.2) (layer "F.Cu") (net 27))
 (segment (start 130.5 86.512941) (end 130.5 86.5) (width 0.2) (layer "F.Cu") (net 27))
 (via (at 128 93.5) (size 0.6) (drill 0.3) (layers "F.Cu" "B.Cu") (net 27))
 (via (at 129.425735 93.425735) (size 0.6) (drill 0.3) (layers "F.Cu" "B.Cu") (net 27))
 (via (at 130.5 86.5) (size 0.6) (drill 0.3) (layers "F.Cu" "B.Cu") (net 27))
 (segment (start 131 85.565686) (end 131 83.565686) (width 0.2) (layer "B.Cu") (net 27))
 (segment (start 128 93.5) (end 129.5 93.5) (width 0.2) (layer "B.Cu") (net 27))
 (segment (start 131.4 80.515) (end 133.115 80.515) (width 0.2) (layer "B.Cu") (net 27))
 (segment (start 129.5 93.5) (end 129.425735 93.425735) (width 0.2) (layer "B.Cu") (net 27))
 (segment (start 131.4 83.165686) (end 131.4 80.515) (width 0.2) (layer "B.Cu") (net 27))
 (segment (start 130.5 86.065686) (end 131 85.565686) (width 0.2) (layer "B.Cu") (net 27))
 (segment (start 131 83.565686) (end 131.4 83.165686) (width 0.2) (layer "B.Cu") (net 27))
 (segment (start 130.5 86.5) (end 130.5 86.065686) (width 0.2) (layer "B.Cu") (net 27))
 (segment (start 129.5 86.5) (end 129 87) (width 0.2) (layer "F.Cu") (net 28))
 (segment (start 129 87) (end 129 92) (width 0.2) (layer "F.Cu") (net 28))
 (segment (start 128.75 95.53875) (end 128.2 96.08875) (width 0.2) (layer "F.Cu") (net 28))
 (segment (start 133.115 77.975) (end 132.49 78.6) (width 0.2) (layer "F.Cu") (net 28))
 (segment (start 129.5 86.5) (end 129.5 84.69) (width 0.2) (layer "F.Cu") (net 28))
 (segment (start 129 92) (end 128.75 92.25) (width 0.2) (layer "F.Cu") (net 28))
 (segment (start 129.5 84.69) (end 129.31 84.5) (width 0.2) (layer "F.Cu") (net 28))
 (segment (start 128.75 92.25) (end 128.75 95.53875) (width 0.2) (layer "F.Cu") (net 28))
 (via (at 129.5 86.5) (size 0.6) (drill 0.3) (layers "F.Cu" "B.Cu") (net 28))
 (segment (start 129.5 86.5) (end 130.5 85.5) (width 0.2) (layer "B.Cu") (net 28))
 (segment (start 131 83) (end 131 78) (width 0.2) (layer "B.Cu") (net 28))
 (segment (start 130.5 85.5) (end 130.5 83.5) (width 0.2) (layer "B.Cu") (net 28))
 (segment (start 131 78) (end 131.025 77.975) (width 0.2) (layer "B.Cu") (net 28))
 (segment (start 131.025 77.975) (end 133.115 77.975) (width 0.2) (layer "B.Cu") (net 28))
 (segment (start 130.5 83.5) (end 131 83) (width 0.2) (layer "B.Cu") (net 28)))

